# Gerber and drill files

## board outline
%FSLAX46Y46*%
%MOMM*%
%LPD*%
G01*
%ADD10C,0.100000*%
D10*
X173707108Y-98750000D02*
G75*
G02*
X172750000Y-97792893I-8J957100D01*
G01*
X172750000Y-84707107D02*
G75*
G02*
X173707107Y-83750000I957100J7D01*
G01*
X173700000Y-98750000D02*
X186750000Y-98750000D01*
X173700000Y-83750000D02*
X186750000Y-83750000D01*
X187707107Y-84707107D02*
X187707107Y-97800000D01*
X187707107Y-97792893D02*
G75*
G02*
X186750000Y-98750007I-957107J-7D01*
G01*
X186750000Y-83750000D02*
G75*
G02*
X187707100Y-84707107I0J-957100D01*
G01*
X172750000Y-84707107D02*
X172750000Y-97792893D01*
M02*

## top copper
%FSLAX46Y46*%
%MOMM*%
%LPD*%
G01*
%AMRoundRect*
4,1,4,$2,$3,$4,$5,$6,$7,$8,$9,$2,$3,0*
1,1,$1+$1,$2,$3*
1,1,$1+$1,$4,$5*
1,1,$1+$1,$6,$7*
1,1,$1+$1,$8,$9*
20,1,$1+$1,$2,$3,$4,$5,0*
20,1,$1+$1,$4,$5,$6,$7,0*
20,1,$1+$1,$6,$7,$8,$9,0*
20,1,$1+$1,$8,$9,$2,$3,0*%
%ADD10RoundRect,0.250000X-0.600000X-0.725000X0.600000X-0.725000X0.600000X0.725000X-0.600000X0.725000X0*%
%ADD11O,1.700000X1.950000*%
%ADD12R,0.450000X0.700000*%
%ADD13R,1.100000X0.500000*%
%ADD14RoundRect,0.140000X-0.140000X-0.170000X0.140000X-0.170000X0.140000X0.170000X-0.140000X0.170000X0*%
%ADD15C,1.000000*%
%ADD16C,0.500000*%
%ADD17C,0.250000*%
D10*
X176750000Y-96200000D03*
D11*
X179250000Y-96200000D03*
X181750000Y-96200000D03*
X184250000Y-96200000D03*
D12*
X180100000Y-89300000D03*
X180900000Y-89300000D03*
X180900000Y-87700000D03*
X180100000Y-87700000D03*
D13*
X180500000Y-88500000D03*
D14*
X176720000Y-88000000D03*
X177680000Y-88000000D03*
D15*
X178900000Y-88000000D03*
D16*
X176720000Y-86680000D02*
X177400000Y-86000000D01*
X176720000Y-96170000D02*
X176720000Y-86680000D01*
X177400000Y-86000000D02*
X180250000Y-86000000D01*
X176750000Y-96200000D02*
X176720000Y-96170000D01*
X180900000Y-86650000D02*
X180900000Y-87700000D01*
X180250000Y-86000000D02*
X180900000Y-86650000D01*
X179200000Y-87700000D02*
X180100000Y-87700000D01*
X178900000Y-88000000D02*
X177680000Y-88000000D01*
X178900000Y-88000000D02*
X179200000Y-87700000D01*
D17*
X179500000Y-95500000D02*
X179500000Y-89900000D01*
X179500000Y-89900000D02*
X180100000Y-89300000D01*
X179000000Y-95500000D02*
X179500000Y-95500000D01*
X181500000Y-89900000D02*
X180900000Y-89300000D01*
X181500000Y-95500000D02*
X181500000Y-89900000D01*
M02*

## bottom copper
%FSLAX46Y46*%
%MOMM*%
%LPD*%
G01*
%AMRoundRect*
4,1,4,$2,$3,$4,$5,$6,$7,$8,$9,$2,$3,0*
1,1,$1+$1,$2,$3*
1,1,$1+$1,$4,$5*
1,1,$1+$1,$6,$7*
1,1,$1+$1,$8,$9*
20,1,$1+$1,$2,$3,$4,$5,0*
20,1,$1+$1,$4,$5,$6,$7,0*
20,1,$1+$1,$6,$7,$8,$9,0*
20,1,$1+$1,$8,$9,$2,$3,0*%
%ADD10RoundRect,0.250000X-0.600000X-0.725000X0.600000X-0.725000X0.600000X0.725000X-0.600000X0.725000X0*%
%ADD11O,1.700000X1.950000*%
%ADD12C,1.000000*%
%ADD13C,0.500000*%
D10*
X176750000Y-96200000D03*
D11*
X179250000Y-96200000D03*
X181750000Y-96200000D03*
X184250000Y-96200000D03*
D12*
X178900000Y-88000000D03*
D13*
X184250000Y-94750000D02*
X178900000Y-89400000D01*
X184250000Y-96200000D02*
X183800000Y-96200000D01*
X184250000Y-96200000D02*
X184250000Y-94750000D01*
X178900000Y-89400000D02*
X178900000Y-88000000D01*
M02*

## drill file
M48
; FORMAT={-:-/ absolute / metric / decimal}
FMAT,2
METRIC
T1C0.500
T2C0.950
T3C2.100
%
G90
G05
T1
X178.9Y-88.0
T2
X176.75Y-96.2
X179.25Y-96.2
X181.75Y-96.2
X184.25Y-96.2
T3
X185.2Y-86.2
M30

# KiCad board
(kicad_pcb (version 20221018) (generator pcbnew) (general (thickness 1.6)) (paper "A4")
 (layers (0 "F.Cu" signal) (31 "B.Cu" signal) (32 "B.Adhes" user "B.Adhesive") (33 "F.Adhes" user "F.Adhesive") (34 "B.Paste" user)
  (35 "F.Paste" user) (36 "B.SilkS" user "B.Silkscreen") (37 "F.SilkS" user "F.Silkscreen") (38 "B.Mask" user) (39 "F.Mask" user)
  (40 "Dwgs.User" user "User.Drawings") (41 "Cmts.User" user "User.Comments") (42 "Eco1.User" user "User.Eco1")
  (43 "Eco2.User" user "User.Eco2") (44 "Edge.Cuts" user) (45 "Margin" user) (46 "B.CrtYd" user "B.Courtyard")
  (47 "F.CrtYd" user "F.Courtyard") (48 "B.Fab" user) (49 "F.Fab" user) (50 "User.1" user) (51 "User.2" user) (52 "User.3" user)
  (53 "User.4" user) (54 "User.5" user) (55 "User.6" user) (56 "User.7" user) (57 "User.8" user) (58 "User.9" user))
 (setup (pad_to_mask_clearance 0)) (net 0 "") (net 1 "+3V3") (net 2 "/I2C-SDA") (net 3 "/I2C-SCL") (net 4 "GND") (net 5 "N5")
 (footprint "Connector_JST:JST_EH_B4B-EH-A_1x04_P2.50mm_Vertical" (layer "F.Cu") (at 176.75 96.2)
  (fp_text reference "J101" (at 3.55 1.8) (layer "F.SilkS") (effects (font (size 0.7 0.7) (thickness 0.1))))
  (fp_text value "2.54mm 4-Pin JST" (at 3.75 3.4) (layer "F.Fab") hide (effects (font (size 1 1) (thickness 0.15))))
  (pad "1" thru_hole roundrect (at 0 0) (size 1.7 1.95) (drill 0.95) (layers "*.Cu" "*.Mask") (roundrect_rratio 0.147059) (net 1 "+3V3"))
  (pad "2" thru_hole oval (at 2.5 0) (size 1.7 1.95) (drill 0.95) (layers "*.Cu" "*.Mask") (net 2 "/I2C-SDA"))
  (pad "3" thru_hole oval (at 5 0) (size 1.7 1.95) (drill 0.95) (layers "*.Cu" "*.Mask") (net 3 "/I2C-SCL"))
  (pad "4" thru_hole oval (at 7.5 0) (size 1.7 1.95) (drill 0.95) (layers "*.Cu" "*.Mask") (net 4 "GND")))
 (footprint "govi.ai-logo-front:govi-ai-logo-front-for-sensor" (layer "F.Cu") (at 180.3 92.3)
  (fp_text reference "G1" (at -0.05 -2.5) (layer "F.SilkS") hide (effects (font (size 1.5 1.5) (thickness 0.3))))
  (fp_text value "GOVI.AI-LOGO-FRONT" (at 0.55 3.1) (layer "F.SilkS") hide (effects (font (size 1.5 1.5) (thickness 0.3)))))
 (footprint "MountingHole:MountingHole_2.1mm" (layer "F.Cu") (at 185.2 86.2)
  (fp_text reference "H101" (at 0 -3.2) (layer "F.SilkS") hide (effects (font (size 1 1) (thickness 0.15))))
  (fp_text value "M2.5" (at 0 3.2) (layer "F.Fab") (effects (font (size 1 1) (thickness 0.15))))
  (pad "" np_thru_hole circle (at 0 0) (size 2.1 2.1) (drill 2.1) (layers "*.Cu" "*.Mask")))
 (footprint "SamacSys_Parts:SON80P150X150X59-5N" (layer "F.Cu") (at 180.5 88.5 90)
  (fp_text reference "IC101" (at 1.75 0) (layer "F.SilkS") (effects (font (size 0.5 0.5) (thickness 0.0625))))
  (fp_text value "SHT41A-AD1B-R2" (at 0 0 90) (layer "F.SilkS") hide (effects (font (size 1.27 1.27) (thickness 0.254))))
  (pad "1" smd rect (at -0.8 -0.4 180) (size 0.45 0.7) (layers "F.Cu" "F.Paste" "F.Mask") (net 2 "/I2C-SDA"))
  (pad "2" smd rect (at -0.8 0.4 180) (size 0.45 0.7) (layers "F.Cu" "F.Paste" "F.Mask") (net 3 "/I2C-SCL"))
  (pad "3" smd rect (at 0.8 0.4 180) (size 0.45 0.7) (layers "F.Cu" "F.Paste" "F.Mask") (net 1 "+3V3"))
  (pad "4" smd rect (at 0.8 -0.4 180) (size 0.45 0.7) (layers "F.Cu" "F.Paste" "F.Mask") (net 4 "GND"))
  (pad "5" smd rect (at 0 0 90) (size 0.5 1.1) (layers "F.Cu" "F.Paste" "F.Mask") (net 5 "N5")))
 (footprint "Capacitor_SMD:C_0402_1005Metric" (layer "F.Cu") (at 177.2 88)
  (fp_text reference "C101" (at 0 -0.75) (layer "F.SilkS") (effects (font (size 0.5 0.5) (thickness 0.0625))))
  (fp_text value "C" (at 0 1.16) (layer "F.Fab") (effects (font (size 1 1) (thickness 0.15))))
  (pad "1" smd roundrect (at -0.48 0) (size 0.56 0.62) (layers "F.Cu" "F.Paste" "F.Mask") (roundrect_rratio 0.25) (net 1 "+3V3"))
  (pad "2" smd roundrect (at 0.48 0) (size 0.56 0.62) (layers "F.Cu" "F.Paste" "F.Mask") (roundrect_rratio 0.25) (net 4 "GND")))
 (gr_arc (start 173.707108 98.75) (mid 173.030331 98.46967) (end 172.750001 97.792893) (stroke (width 0.1) (type default))
  (layer "Edge.Cuts"))
 (gr_arc (start 172.75 84.707107) (mid 173.03033 84.03033) (end 173.707107 83.75) (stroke (width 0.1) (type default)) (layer "Edge.Cuts"))
 (gr_line (start 173.7 98.75) (end 186.75 98.75) (stroke (width 0.1) (type default)) (layer "Edge.Cuts"))
 (gr_line (start 173.7 83.75) (end 186.75 83.75) (stroke (width 0.1) (type default)) (layer "Edge.Cuts"))
 (gr_line (start 187.707107 84.707107) (end 187.707107 97.8) (stroke (width 0.1) (type default)) (layer "Edge.Cuts"))
 (gr_arc (start 187.707107 97.792893) (mid 187.426778 98.469671) (end 186.75 98.75) (stroke (width 0.1) (type default)) (layer "Edge.Cuts"))
 (gr_arc (start 186.75 83.75) (mid 187.426777 84.03033) (end 187.707107 84.707107) (stroke (width 0.1) (type default)) (layer "Edge.Cuts"))
 (gr_line (start 172.75 84.707107) (end 172.75 97.792893) (stroke (width 0.1) (type default)) (layer "Edge.Cuts"))
 (segment (start 176.72 86.68) (end 177.4 86) (width 0.5) (layer "F.Cu") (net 1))
 (segment (start 176.72 96.17) (end 176.72 86.68) (width 0.5) (layer "F.Cu") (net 1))
 (segment (start 177.4 86) (end 180.25 86) (width 0.5) (layer "F.Cu") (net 1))
 (segment (start 176.75 96.2) (end 176.72 96.17) (width 0.5) (layer "F.Cu") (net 1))
 (segment (start 180.9 86.65) (end 180.9 87.7) (width 0.5) (layer "F.Cu") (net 1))
 (segment (start 180.25 86) (end 180.9 86.65) (width 0.5) (layer "F.Cu") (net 1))
 (segment (start 179.2 87.7) (end 180.1 87.7) (width 0.5) (layer "F.Cu") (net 4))
 (segment (start 178.9 88) (end 177.68 88) (width 0.5) (layer "F.Cu") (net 4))
 (segment (start 178.9 88) (end 179.2 87.7) (width 0.5) (layer "F.Cu") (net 4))
 (via (at 178.9 88) (size 1) (drill 0.5) (layers "F.Cu" "B.Cu") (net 4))
 (segment (start 184.25 94.75) (end 178.9 89.4) (width 0.5) (layer "B.Cu") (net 4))
 (segment (start 184.25 96.2) (end 183.8 96.2) (width 0.5) (layer "B.Cu") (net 4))
 (segment (start 184.25 96.2) (end 184.25 94.75) (width 0.5) (layer "B.Cu") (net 4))
 (segment (start 178.9 89.4) (end 178.9 88) (width 0.5) (layer "B.Cu") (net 4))
 (segment (start 179.5 95.5) (end 179.5 89.9) (width 0.25) (layer "F.Cu") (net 2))
 (segment (start 179.5 89.9) (end 180.1 89.3) (width 0.25) (layer "F.Cu") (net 2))
 (segment (start 179 95.5) (end 179.5 95.5) (width 0.25) (layer "F.Cu") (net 2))
 (segment (start 181.5 89.9) (end 180.9 89.3) (width 0.25) (layer "F.Cu") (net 3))
 (segment (start 181.5 95.5) (end 181.5 89.9) (width 0.25) (layer "F.Cu") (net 3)))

